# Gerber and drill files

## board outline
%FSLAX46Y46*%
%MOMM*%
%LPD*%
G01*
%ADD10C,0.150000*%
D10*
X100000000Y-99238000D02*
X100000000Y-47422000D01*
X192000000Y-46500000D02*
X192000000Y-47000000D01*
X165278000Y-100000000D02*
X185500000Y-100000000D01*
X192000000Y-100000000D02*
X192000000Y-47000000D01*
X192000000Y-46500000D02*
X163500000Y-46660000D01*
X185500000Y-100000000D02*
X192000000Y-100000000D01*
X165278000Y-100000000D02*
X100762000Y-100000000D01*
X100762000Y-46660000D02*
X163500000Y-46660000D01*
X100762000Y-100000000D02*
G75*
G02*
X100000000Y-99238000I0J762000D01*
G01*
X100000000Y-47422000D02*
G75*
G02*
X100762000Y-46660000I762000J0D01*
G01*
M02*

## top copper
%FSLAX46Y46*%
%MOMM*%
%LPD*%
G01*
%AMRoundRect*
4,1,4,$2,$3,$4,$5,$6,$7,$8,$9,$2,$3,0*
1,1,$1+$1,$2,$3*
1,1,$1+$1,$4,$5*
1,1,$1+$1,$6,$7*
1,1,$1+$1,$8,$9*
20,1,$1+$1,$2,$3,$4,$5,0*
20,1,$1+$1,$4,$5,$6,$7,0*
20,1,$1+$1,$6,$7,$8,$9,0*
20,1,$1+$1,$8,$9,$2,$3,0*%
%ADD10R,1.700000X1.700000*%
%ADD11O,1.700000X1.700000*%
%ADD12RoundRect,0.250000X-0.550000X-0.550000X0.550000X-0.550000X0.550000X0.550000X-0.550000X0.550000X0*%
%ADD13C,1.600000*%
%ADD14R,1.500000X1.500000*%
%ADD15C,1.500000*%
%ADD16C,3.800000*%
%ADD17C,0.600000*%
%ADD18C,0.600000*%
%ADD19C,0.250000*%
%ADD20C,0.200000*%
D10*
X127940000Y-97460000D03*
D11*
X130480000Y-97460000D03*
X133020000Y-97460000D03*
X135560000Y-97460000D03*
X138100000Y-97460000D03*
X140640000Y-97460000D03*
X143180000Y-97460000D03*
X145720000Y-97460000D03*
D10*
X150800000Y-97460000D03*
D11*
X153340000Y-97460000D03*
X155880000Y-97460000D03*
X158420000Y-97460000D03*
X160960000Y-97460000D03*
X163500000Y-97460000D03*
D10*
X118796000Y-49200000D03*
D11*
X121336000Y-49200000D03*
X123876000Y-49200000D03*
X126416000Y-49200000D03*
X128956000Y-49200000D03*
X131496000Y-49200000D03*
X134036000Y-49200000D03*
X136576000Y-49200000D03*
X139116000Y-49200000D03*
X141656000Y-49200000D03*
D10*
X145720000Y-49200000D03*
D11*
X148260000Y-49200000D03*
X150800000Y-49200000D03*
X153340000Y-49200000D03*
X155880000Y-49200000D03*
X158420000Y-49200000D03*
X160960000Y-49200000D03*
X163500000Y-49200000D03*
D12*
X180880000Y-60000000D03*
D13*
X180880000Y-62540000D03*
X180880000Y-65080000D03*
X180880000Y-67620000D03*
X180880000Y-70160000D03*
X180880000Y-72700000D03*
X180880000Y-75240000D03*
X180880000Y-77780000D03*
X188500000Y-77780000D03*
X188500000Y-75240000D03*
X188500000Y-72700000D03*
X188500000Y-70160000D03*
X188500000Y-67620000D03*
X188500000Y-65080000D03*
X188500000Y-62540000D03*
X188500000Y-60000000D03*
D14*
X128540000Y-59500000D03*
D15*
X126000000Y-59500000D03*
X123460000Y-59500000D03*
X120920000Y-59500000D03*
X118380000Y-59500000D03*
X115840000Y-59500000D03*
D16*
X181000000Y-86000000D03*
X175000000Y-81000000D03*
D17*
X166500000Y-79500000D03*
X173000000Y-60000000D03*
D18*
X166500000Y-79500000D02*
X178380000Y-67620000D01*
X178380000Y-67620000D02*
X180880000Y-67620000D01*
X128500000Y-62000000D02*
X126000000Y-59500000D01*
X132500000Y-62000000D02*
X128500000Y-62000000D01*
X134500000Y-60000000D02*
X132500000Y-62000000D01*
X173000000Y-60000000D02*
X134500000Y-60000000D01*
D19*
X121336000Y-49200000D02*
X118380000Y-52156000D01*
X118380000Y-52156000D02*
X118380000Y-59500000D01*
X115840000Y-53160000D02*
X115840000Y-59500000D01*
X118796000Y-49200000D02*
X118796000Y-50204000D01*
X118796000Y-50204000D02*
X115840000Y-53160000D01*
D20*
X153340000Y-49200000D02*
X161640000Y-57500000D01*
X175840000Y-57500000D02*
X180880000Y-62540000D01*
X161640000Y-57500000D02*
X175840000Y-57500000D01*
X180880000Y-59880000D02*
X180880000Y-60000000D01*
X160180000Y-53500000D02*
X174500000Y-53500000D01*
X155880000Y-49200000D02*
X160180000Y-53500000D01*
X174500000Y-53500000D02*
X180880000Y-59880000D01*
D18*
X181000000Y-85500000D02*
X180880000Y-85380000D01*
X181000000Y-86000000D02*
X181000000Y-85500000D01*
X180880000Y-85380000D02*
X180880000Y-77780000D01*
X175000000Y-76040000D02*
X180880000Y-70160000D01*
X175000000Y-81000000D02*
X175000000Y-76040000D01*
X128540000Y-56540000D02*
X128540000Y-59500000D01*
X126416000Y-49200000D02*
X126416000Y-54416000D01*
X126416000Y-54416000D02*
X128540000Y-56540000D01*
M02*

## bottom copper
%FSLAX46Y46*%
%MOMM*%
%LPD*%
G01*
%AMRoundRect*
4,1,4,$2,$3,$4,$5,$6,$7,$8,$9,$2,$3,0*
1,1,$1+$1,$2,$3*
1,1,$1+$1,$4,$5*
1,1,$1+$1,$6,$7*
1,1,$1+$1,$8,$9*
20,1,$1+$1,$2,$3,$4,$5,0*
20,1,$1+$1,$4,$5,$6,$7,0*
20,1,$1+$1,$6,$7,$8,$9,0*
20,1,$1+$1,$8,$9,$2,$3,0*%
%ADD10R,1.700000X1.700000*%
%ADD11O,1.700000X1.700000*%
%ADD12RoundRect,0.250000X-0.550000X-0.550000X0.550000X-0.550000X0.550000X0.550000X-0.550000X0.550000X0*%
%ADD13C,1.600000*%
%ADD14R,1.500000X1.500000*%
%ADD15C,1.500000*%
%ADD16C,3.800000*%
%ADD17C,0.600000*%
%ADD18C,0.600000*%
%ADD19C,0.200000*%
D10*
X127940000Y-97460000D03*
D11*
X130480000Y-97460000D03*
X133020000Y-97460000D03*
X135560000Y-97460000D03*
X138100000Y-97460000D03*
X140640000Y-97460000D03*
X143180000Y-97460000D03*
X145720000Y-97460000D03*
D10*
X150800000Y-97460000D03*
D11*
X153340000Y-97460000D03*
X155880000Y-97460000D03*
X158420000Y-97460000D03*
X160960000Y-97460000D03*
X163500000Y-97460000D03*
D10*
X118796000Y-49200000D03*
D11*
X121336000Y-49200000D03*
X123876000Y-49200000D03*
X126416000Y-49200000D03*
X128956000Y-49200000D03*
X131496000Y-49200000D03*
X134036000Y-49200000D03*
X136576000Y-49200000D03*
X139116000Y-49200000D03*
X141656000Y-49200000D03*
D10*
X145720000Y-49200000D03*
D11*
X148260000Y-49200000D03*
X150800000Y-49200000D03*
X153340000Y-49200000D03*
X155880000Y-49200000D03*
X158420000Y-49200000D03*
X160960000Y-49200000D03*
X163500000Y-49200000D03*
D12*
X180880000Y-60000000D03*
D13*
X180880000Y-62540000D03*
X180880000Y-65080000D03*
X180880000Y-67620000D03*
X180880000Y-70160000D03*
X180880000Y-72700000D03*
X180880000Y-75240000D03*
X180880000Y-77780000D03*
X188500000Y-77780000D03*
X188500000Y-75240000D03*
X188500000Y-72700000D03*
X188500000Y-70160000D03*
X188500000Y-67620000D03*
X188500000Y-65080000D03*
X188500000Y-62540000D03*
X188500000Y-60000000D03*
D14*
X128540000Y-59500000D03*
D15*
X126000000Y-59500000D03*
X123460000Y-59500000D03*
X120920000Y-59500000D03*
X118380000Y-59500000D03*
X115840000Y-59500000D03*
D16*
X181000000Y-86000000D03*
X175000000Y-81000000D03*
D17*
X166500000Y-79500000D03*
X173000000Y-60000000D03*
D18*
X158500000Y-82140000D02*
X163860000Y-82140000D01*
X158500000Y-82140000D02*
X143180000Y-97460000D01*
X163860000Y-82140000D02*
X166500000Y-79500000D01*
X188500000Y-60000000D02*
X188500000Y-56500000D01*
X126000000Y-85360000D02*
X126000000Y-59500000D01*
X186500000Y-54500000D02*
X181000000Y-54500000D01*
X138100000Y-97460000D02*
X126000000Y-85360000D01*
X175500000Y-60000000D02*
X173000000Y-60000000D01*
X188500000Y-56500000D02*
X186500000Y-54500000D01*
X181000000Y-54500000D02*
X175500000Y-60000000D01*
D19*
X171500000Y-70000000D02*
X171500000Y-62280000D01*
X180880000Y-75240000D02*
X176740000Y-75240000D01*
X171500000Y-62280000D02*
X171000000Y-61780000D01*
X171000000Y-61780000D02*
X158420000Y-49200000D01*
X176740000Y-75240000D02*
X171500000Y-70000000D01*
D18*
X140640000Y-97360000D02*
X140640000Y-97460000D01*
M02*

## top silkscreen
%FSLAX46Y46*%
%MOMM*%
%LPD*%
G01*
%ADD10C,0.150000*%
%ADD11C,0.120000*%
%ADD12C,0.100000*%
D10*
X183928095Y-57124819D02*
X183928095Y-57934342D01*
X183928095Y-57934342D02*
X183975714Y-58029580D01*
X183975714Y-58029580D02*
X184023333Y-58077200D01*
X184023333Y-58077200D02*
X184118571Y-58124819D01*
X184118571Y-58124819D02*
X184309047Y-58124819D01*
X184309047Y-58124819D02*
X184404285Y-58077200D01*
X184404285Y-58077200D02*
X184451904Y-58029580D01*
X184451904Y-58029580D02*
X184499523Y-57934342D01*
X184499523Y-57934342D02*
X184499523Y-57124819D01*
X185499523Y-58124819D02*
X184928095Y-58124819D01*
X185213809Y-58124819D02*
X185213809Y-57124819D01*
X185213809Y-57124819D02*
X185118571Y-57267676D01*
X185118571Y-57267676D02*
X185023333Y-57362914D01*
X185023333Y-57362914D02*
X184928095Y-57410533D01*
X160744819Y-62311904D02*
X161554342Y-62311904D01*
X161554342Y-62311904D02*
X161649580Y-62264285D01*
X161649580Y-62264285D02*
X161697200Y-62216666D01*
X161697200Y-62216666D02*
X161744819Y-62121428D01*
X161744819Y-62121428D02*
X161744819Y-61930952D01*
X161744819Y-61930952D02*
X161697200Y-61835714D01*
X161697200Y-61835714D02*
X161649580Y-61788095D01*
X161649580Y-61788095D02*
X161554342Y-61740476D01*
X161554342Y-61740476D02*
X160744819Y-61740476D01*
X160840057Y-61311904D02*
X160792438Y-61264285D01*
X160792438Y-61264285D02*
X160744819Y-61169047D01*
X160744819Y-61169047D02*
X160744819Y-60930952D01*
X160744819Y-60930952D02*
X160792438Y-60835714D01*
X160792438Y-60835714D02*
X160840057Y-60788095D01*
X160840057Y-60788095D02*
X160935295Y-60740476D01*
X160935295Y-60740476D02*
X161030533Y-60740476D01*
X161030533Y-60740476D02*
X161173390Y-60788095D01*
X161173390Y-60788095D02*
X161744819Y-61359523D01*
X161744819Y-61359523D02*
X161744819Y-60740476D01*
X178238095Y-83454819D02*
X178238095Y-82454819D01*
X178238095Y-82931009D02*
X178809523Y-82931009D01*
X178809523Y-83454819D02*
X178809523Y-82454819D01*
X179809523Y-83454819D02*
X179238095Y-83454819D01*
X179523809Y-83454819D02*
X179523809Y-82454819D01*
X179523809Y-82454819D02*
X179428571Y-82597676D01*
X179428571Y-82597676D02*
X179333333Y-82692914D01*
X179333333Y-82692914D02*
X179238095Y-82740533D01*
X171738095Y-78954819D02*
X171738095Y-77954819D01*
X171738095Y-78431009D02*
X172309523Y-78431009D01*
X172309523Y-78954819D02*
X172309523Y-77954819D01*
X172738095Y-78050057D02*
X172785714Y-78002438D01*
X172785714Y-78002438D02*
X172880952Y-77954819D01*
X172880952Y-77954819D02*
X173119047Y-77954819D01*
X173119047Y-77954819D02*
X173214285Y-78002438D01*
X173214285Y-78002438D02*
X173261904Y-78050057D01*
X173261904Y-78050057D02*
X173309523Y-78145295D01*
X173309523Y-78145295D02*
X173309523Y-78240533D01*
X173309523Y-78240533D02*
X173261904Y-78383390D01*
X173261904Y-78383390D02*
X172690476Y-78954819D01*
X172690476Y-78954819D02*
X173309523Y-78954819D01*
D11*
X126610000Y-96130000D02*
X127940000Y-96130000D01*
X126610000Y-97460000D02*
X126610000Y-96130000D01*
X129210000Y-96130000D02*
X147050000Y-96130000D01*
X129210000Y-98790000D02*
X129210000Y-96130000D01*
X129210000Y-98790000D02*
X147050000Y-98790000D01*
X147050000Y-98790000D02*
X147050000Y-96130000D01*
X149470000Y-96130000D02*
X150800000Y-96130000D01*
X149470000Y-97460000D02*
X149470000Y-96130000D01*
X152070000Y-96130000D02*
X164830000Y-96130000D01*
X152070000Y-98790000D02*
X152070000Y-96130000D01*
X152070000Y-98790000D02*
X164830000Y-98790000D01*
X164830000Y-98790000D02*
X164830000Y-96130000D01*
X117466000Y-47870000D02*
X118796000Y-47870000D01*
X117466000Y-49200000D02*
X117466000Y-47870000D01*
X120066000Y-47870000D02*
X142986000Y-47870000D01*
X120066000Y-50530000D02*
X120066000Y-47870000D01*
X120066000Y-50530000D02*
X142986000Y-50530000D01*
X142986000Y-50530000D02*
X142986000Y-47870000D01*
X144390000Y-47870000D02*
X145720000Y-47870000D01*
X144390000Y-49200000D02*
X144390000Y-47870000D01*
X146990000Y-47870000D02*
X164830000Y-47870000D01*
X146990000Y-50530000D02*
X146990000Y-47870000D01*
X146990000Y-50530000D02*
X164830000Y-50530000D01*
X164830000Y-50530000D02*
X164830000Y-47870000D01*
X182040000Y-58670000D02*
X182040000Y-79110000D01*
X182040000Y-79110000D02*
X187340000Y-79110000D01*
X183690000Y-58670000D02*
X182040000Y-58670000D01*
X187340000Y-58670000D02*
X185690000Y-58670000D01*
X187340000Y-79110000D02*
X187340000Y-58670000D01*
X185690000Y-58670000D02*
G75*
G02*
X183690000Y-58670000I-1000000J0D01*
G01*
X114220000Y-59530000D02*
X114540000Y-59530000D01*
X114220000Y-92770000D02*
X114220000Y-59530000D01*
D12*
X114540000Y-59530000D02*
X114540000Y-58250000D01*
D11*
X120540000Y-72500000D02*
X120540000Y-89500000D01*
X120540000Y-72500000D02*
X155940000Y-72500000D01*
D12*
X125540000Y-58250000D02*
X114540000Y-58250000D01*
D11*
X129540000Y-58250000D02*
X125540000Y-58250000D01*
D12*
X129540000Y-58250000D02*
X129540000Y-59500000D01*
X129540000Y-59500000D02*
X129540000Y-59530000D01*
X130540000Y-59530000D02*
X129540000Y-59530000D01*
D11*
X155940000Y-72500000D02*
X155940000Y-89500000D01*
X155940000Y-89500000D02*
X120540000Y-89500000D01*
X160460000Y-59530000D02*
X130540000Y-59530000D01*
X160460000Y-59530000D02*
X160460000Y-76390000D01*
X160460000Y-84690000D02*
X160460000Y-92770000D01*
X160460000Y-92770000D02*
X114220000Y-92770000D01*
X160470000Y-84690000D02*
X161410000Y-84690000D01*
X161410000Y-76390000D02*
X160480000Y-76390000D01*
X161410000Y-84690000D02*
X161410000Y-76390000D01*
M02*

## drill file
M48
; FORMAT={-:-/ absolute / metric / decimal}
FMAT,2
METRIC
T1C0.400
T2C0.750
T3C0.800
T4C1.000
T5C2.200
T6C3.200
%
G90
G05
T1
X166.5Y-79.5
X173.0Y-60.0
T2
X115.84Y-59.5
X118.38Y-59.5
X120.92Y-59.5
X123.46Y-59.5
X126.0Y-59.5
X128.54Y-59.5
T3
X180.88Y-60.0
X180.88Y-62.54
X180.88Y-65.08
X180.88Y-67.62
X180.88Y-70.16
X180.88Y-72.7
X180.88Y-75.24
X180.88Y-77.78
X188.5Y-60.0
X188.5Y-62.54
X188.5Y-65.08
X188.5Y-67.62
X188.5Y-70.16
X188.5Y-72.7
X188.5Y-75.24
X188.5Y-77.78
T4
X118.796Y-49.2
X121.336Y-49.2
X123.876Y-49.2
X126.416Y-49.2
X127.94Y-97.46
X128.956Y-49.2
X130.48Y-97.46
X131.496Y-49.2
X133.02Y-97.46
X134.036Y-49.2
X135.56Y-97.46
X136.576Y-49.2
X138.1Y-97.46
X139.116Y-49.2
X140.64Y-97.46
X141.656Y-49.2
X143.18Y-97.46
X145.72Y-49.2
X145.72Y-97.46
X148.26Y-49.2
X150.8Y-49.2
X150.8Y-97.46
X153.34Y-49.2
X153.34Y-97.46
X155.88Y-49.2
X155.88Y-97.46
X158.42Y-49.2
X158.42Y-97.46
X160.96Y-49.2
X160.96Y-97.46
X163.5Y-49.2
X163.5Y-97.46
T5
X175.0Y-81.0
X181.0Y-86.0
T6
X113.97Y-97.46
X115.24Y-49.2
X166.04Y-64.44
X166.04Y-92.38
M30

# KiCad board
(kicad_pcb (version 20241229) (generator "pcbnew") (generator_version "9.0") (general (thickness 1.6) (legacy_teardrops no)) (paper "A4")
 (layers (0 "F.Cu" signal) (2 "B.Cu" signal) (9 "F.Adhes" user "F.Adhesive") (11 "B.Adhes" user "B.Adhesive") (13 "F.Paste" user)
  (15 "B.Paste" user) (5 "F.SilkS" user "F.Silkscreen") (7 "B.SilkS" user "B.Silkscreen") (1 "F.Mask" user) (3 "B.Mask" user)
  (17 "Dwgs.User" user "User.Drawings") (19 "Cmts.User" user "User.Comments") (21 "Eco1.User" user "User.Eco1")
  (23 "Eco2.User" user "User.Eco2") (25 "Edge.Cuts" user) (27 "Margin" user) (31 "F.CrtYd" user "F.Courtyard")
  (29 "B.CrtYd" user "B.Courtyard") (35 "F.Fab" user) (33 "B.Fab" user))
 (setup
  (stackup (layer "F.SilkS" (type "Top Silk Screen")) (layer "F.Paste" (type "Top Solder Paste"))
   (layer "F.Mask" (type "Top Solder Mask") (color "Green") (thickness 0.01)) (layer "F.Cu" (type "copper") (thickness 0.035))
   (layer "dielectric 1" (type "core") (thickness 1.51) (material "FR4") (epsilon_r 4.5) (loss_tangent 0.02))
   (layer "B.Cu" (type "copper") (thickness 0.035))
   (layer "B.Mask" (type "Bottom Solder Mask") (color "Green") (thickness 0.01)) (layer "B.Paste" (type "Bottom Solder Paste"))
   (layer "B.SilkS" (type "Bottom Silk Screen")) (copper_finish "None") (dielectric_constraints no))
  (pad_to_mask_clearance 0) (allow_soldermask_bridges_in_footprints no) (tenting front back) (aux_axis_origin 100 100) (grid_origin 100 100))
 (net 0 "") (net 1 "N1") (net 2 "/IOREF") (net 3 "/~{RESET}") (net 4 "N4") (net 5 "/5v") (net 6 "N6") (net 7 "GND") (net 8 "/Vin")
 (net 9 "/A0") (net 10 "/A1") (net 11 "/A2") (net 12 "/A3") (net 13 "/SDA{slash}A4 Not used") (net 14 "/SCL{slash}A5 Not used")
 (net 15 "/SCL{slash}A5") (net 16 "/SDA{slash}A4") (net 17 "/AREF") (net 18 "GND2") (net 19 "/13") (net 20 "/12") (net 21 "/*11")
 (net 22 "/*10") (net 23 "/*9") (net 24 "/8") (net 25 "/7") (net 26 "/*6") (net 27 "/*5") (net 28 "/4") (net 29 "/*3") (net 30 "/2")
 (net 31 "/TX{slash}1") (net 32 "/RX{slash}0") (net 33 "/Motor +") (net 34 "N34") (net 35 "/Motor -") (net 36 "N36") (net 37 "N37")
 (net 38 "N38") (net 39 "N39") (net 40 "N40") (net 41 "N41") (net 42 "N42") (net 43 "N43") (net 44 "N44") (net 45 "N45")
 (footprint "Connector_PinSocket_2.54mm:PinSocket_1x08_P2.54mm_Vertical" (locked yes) (layer "F.Cu") (at 127.94 97.46 90)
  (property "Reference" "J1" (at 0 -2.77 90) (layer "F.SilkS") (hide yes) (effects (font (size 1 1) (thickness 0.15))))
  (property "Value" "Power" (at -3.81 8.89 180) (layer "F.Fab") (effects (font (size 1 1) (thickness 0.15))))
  (fp_line (start 1.33 -1.33) (end 1.33 0) (stroke (width 0.12) (type solid)) (layer "F.SilkS"))
  (fp_line (start 0 -1.33) (end 1.33 -1.33) (stroke (width 0.12) (type solid)) (layer "F.SilkS"))
  (fp_line (start 1.33 1.27) (end 1.33 19.11) (stroke (width 0.12) (type solid)) (layer "F.SilkS"))
  (fp_line (start -1.33 1.27) (end 1.33 1.27) (stroke (width 0.12) (type solid)) (layer "F.SilkS"))
  (fp_line (start -1.33 1.27) (end -1.33 19.11) (stroke (width 0.12) (type solid)) (layer "F.SilkS"))
  (fp_line (start -1.33 19.11) (end 1.33 19.11) (stroke (width 0.12) (type solid)) (layer "F.SilkS"))
  (pad "1" thru_hole rect (at 0 0 90) (size 1.7 1.7) (drill 1) (layers "*.Cu" "*.Mask") (remove_unused_layers no) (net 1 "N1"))
  (pad "2" thru_hole oval (at 0 2.54 90) (size 1.7 1.7) (drill 1) (layers "*.Cu" "*.Mask") (remove_unused_layers no) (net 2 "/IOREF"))
  (pad "3" thru_hole oval (at 0 5.08 90) (size 1.7 1.7) (drill 1) (layers "*.Cu" "*.Mask") (remove_unused_layers no) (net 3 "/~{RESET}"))
  (pad "4" thru_hole oval (at 0 7.62 90) (size 1.7 1.7) (drill 1) (layers "*.Cu" "*.Mask") (remove_unused_layers no) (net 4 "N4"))
  (pad "5" thru_hole oval (at 0 10.16 90) (size 1.7 1.7) (drill 1) (layers "*.Cu" "*.Mask") (remove_unused_layers no) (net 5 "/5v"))
  (pad "6" thru_hole oval (at 0 12.7 90) (size 1.7 1.7) (drill 1) (layers "*.Cu" "*.Mask") (remove_unused_layers no) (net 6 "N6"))
  (pad "7" thru_hole oval (at 0 15.24 90) (size 1.7 1.7) (drill 1) (layers "*.Cu" "*.Mask") (remove_unused_layers no) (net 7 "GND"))
  (pad "8" thru_hole oval (at 0 17.78 90) (size 1.7 1.7) (drill 1) (layers "*.Cu" "*.Mask") (remove_unused_layers no) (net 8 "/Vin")))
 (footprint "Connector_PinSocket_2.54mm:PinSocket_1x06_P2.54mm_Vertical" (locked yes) (layer "F.Cu") (at 150.8 97.46 90)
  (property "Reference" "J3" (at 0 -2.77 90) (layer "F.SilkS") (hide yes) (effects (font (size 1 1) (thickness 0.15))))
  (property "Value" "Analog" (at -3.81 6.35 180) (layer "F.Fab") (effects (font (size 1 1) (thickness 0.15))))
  (fp_line (start 1.33 -1.33) (end 1.33 0) (stroke (width 0.12) (type solid)) (layer "F.SilkS"))
  (fp_line (start 0 -1.33) (end 1.33 -1.33) (stroke (width 0.12) (type solid)) (layer "F.SilkS"))
  (fp_line (start 1.33 1.27) (end 1.33 14.03) (stroke (width 0.12) (type solid)) (layer "F.SilkS"))
  (fp_line (start -1.33 1.27) (end 1.33 1.27) (stroke (width 0.12) (type solid)) (layer "F.SilkS"))
  (fp_line (start -1.33 1.27) (end -1.33 14.03) (stroke (width 0.12) (type solid)) (layer "F.SilkS"))
  (fp_line (start -1.33 14.03) (end 1.33 14.03) (stroke (width 0.12) (type solid)) (layer "F.SilkS"))
  (pad "1" thru_hole rect (at 0 0 90) (size 1.7 1.7) (drill 1) (layers "*.Cu" "*.Mask") (remove_unused_layers no) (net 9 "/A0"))
  (pad "2" thru_hole oval (at 0 2.54 90) (size 1.7 1.7) (drill 1) (layers "*.Cu" "*.Mask") (remove_unused_layers no) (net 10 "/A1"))
  (pad "3" thru_hole oval (at 0 5.08 90) (size 1.7 1.7) (drill 1) (layers "*.Cu" "*.Mask") (remove_unused_layers no) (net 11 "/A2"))
  (pad "4" thru_hole oval (at 0 7.62 90) (size 1.7 1.7) (drill 1) (layers "*.Cu" "*.Mask") (remove_unused_layers no) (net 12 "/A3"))
  (pad "5" thru_hole oval (at 0 10.16 90) (size 1.7 1.7) (drill 1) (layers "*.Cu" "*.Mask") (remove_unused_layers no)
   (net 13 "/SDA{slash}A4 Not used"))
  (pad "6" thru_hole oval (at 0 12.7 90) (size 1.7 1.7) (drill 1) (layers "*.Cu" "*.Mask") (remove_unused_layers no)
   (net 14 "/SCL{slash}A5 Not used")))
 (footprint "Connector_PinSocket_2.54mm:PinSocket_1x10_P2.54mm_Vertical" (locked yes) (layer "F.Cu") (at 118.796 49.2 90)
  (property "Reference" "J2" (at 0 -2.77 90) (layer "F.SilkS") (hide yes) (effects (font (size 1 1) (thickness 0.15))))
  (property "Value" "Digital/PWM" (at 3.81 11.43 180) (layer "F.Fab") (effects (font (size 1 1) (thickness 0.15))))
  (fp_line (start 1.33 -1.33) (end 1.33 0) (stroke (width 0.12) (type solid)) (layer "F.SilkS"))
  (fp_line (start 0 -1.33) (end 1.33 -1.33) (stroke (width 0.12) (type solid)) (layer "F.SilkS"))
  (fp_line (start 1.33 1.27) (end 1.33 24.19) (stroke (width 0.12) (type solid)) (layer "F.SilkS"))
  (fp_line (start -1.33 1.27) (end 1.33 1.27) (stroke (width 0.12) (type solid)) (layer "F.SilkS"))
  (fp_line (start -1.33 1.27) (end -1.33 24.19) (stroke (width 0.12) (type solid)) (layer "F.SilkS"))
  (fp_line (start -1.33 24.19) (end 1.33 24.19) (stroke (width 0.12) (type solid)) (layer "F.SilkS"))
  (pad "1" thru_hole rect (at 0 0 90) (size 1.7 1.7) (drill 1) (layers "*.Cu" "*.Mask") (remove_unused_layers no) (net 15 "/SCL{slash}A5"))
  (pad "2" thru_hole oval (at 0 2.54 90) (size 1.7 1.7) (drill 1) (layers "*.Cu" "*.Mask") (remove_unused_layers no)
   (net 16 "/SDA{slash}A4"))
  (pad "3" thru_hole oval (at 0 5.08 90) (size 1.7 1.7) (drill 1) (layers "*.Cu" "*.Mask") (remove_unused_layers no) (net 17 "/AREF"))
  (pad "4" thru_hole oval (at 0 7.62 90) (size 1.7 1.7) (drill 1) (layers "*.Cu" "*.Mask") (remove_unused_layers no) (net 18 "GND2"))
  (pad "5" thru_hole oval (at 0 10.16 90) (size 1.7 1.7) (drill 1) (layers "*.Cu" "*.Mask") (remove_unused_layers no) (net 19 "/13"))
  (pad "6" thru_hole oval (at 0 12.7 90) (size 1.7 1.7) (drill 1) (layers "*.Cu" "*.Mask") (remove_unused_layers no) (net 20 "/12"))
  (pad "7" thru_hole oval (at 0 15.24 90) (size 1.7 1.7) (drill 1) (layers "*.Cu" "*.Mask") (remove_unused_layers no) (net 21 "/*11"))
  (pad "8" thru_hole oval (at 0 17.78 90) (size 1.7 1.7) (drill 1) (layers "*.Cu" "*.Mask") (remove_unused_layers no) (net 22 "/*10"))
  (pad "9" thru_hole oval (at 0 20.32 90) (size 1.7 1.7) (drill 1) (layers "*.Cu" "*.Mask") (remove_unused_layers no) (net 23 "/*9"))
  (pad "10" thru_hole oval (at 0 22.86 90) (size 1.7 1.7) (drill 1) (layers "*.Cu" "*.Mask") (remove_unused_layers no) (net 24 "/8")))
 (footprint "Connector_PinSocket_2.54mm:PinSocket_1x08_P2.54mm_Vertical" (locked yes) (layer "F.Cu") (at 145.72 49.2 90)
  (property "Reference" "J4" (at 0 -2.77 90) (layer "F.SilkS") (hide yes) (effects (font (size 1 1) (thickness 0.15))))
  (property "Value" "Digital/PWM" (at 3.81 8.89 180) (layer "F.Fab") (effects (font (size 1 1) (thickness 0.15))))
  (fp_line (start 1.33 -1.33) (end 1.33 0) (stroke (width 0.12) (type solid)) (layer "F.SilkS"))
  (fp_line (start 0 -1.33) (end 1.33 -1.33) (stroke (width 0.12) (type solid)) (layer "F.SilkS"))
  (fp_line (start 1.33 1.27) (end 1.33 19.11) (stroke (width 0.12) (type solid)) (layer "F.SilkS"))
  (fp_line (start -1.33 1.27) (end 1.33 1.27) (stroke (width 0.12) (type solid)) (layer "F.SilkS"))
  (fp_line (start -1.33 1.27) (end -1.33 19.11) (stroke (width 0.12) (type solid)) (layer "F.SilkS"))
  (fp_line (start -1.33 19.11) (end 1.33 19.11) (stroke (width 0.12) (type solid)) (layer "F.SilkS"))
  (pad "1" thru_hole rect (at 0 0 90) (size 1.7 1.7) (drill 1) (layers "*.Cu" "*.Mask") (remove_unused_layers no) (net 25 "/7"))
  (pad "2" thru_hole oval (at 0 2.54 90) (size 1.7 1.7) (drill 1) (layers "*.Cu" "*.Mask") (remove_unused_layers no) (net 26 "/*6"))
  (pad "3" thru_hole oval (at 0 5.08 90) (size 1.7 1.7) (drill 1) (layers "*.Cu" "*.Mask") (remove_unused_layers no) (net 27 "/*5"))
  (pad "4" thru_hole oval (at 0 7.62 90) (size 1.7 1.7) (drill 1) (layers "*.Cu" "*.Mask") (remove_unused_layers no) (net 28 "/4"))
  (pad "5" thru_hole oval (at 0 10.16 90) (size 1.7 1.7) (drill 1) (layers "*.Cu" "*.Mask") (remove_unused_layers no) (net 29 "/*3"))
  (pad "6" thru_hole oval (at 0 12.7 90) (size 1.7 1.7) (drill 1) (layers "*.Cu" "*.Mask") (remove_unused_layers no) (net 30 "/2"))
  (pad "7" thru_hole oval (at 0 15.24 90) (size 1.7 1.7) (drill 1) (layers "*.Cu" "*.Mask") (remove_unused_layers no) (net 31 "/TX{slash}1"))
  (pad "8" thru_hole oval (at 0 17.78 90) (size 1.7 1.7) (drill 1) (layers "*.Cu" "*.Mask") (remove_unused_layers no) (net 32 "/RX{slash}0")))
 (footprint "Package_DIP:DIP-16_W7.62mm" (layer "F.Cu") (at 180.88 60)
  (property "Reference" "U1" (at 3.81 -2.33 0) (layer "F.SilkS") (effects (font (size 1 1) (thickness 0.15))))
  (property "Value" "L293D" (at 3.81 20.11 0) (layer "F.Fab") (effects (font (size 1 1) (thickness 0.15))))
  (fp_line (start 1.16 -1.33) (end 1.16 19.11) (stroke (width 0.12) (type solid)) (layer "F.SilkS"))
  (fp_line (start 1.16 19.11) (end 6.46 19.11) (stroke (width 0.12) (type solid)) (layer "F.SilkS"))
  (fp_line (start 2.81 -1.33) (end 1.16 -1.33) (stroke (width 0.12) (type solid)) (layer "F.SilkS"))
  (fp_line (start 6.46 -1.33) (end 4.81 -1.33) (stroke (width 0.12) (type solid)) (layer "F.SilkS"))
  (fp_line (start 6.46 19.11) (end 6.46 -1.33) (stroke (width 0.12) (type solid)) (layer "F.SilkS"))
  (fp_arc (start 4.81 -1.33) (mid 3.81 -0.33) (end 2.81 -1.33) (stroke (width 0.12) (type solid)) (layer "F.SilkS"))
  (pad "1" thru_hole roundrect (at 0 0) (size 1.6 1.6) (drill 0.8) (layers "*.Cu" "*.Mask") (remove_unused_layers no)
   (roundrect_rratio 0.15625) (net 29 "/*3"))
  (pad "2" thru_hole circle (at 0 2.54) (size 1.6 1.6) (drill 0.8) (layers "*.Cu" "*.Mask") (remove_unused_layers no) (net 28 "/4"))
  (pad "3" thru_hole circle (at 0 5.08) (size 1.6 1.6) (drill 0.8) (layers "*.Cu" "*.Mask") (remove_unused_layers no) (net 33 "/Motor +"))
  (pad "4" thru_hole circle (at 0 7.62) (size 1.6 1.6) (drill 0.8) (layers "*.Cu" "*.Mask") (remove_unused_layers no) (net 7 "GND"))
  (pad "5" thru_hole circle (at 0 10.16) (size 1.6 1.6) (drill 0.8) (layers "*.Cu" "*.Mask") (remove_unused_layers no) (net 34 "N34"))
  (pad "6" thru_hole circle (at 0 12.7) (size 1.6 1.6) (drill 0.8) (layers "*.Cu" "*.Mask") (remove_unused_layers no) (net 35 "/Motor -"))
  (pad "7" thru_hole circle (at 0 15.24) (size 1.6 1.6) (drill 0.8) (layers "*.Cu" "*.Mask") (remove_unused_layers no) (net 30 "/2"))
  (pad "8" thru_hole circle (at 0 17.78) (size 1.6 1.6) (drill 0.8) (layers "*.Cu" "*.Mask") (remove_unused_layers no) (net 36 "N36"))
  (pad "9" thru_hole circle (at 7.62 17.78) (size 1.6 1.6) (drill 0.8) (layers "*.Cu" "*.Mask") (remove_unused_layers no) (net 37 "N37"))
  (pad "10" thru_hole circle (at 7.62 15.24) (size 1.6 1.6) (drill 0.8) (layers "*.Cu" "*.Mask") (remove_unused_layers no) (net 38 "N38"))
  (pad "11" thru_hole circle (at 7.62 12.7) (size 1.6 1.6) (drill 0.8) (layers "*.Cu" "*.Mask") (remove_unused_layers no) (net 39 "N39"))
  (pad "12" thru_hole circle (at 7.62 10.16) (size 1.6 1.6) (drill 0.8) (layers "*.Cu" "*.Mask") (remove_unused_layers no) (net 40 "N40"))
  (pad "13" thru_hole circle (at 7.62 7.62) (size 1.6 1.6) (drill 0.8) (layers "*.Cu" "*.Mask") (remove_unused_layers no) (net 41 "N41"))
  (pad "14" thru_hole circle (at 7.62 5.08) (size 1.6 1.6) (drill 0.8) (layers "*.Cu" "*.Mask") (remove_unused_layers no) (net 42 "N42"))
  (pad "15" thru_hole circle (at 7.62 2.54) (size 1.6 1.6) (drill 0.8) (layers "*.Cu" "*.Mask") (remove_unused_layers no) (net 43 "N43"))
  (pad "16" thru_hole circle (at 7.62 0) (size 1.6 1.6) (drill 0.8) (layers "*.Cu" "*.Mask") (remove_unused_layers no) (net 5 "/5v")))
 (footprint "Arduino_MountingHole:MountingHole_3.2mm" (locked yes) (layer "F.Cu") (at 115.24 49.2)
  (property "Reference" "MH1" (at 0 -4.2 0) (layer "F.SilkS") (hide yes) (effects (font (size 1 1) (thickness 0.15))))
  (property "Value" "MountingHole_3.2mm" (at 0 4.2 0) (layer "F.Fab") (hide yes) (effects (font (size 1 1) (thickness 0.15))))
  (pad "" np_thru_hole circle (at 0 0) (size 3.2 3.2) (drill 3.2) (layers "*.Cu" "*.Mask")))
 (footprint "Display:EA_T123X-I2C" (layer "F.Cu") (at 128.54 59.5 -90)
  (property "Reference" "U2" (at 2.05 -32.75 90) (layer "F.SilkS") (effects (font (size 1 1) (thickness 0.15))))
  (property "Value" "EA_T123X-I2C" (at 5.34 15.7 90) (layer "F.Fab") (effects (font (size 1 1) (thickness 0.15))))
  (fp_line (start 0.03 14.32) (end 0.03 14) (stroke (width 0.12) (type solid)) (layer "F.SilkS"))
  (fp_line (start 33.27 14.32) (end 0.03 14.32) (stroke (width 0.12) (type solid)) (layer "F.SilkS"))
  (fp_line (start 0.03 14) (end -1.25 14) (stroke (width 0.1) (type default)) (layer "F.SilkS"))
  (fp_line (start 13 8) (end 30 8) (stroke (width 0.12) (type solid)) (layer "F.SilkS"))
  (fp_line (start 13 8) (end 13 -27.4) (stroke (width 0.12) (type solid)) (layer "F.SilkS"))
  (fp_line (start -1.25 3) (end -1.25 14) (stroke (width 0.1) (type default)) (layer "F.SilkS"))
  (fp_line (start -1.25 -1) (end -1.25 3) (stroke (width 0.12) (type solid)) (layer "F.SilkS"))
  (fp_line (start -1.25 -1) (end 0 -1) (stroke (width 0.1) (type default)) (layer "F.SilkS"))
  (fp_line (start 0 -1) (end 0.03 -1) (stroke (width 0.1) (type default)) (layer "F.SilkS"))
  (fp_line (start 0.03 -2) (end 0.03 -1) (stroke (width 0.1) (type default)) (layer "F.SilkS"))
  (fp_line (start 13 -27.4) (end 30 -27.4) (stroke (width 0.12) (type solid)) (layer "F.SilkS"))
  (fp_line (start 30 -27.4) (end 30 8) (stroke (width 0.12) (type solid)) (layer "F.SilkS"))
  (fp_line (start 0.03 -31.92) (end 0.03 -2) (stroke (width 0.12) (type solid)) (layer "F.SilkS"))
  (fp_line (start 0.03 -31.92) (end 16.89 -31.92) (stroke (width 0.12) (type solid)) (layer "F.SilkS"))
  (fp_line (start 25.19 -31.92) (end 33.27 -31.92) (stroke (width 0.12) (type solid)) (layer "F.SilkS"))
  (fp_line (start 33.27 -31.92) (end 33.27 14.32) (stroke (width 0.12) (type solid)) (layer "F.SilkS"))
  (fp_line (start 25.19 -31.93) (end 25.19 -32.87) (stroke (width 0.12) (type solid)) (layer "F.SilkS"))
  (fp_line (start 16.89 -32.87) (end 16.89 -31.94) (stroke (width 0.12) (type solid)) (layer "F.SilkS"))
  (fp_line (start 25.19 -32.87) (end 16.89 -32.87) (stroke (width 0.12) (type solid)) (layer "F.SilkS"))
  (pad "1" thru_hole rect (at 0 0 270) (size 1.5 1.5) (drill 0.75) (layers "*.Cu" "*.Mask") (remove_unused_layers no) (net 18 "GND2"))
  (pad "2" thru_hole circle (at 0 2.54 270) (size 1.5 1.5) (drill 0.75) (layers "*.Cu" "*.Mask") (remove_unused_layers no) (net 5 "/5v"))
  (pad "3" thru_hole circle (at 0 5.08 270) (size 1.5 1.5) (drill 0.75) (layers "*.Cu" "*.Mask") (remove_unused_layers no) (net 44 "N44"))
  (pad "4" thru_hole circle (at 0 7.62 270) (size 1.5 1.5) (drill 0.75) (layers "*.Cu" "*.Mask") (remove_unused_layers no) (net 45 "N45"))
  (pad "5" thru_hole circle (at 0 10.16 270) (size 1.5 1.5) (drill 0.75) (layers "*.Cu" "*.Mask") (remove_unused_layers no)
   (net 16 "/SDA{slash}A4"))
  (pad "6" thru_hole circle (at 0 12.7 270) (size 1.5 1.5) (drill 0.75) (layers "*.Cu" "*.Mask") (remove_unused_layers no)
   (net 15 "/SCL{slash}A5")))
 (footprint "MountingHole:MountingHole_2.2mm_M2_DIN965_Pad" (layer "F.Cu") (at 181 86)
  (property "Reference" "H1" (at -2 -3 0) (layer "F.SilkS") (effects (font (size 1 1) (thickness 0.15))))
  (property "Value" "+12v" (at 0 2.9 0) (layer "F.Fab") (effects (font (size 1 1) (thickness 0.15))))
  (pad "1" thru_hole circle (at 0 0) (size 3.8 3.8) (drill 2.2) (layers "*.Cu" "*.Mask") (remove_unused_layers no) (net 36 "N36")))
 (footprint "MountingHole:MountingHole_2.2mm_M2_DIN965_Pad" (layer "F.Cu") (at 175 81)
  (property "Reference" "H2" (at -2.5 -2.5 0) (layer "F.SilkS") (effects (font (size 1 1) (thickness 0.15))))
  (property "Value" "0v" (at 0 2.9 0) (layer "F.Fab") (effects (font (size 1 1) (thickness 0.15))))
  (pad "1" thru_hole circle (at 0 0) (size 3.8 3.8) (drill 2.2) (layers "*.Cu" "*.Mask") (remove_unused_layers no) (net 34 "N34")))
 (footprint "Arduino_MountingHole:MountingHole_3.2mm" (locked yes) (layer "F.Cu") (at 113.97 97.46)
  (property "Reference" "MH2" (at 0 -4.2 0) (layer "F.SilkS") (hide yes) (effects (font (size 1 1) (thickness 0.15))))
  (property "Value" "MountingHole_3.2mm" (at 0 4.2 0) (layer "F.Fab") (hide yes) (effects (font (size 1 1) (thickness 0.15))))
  (pad "" np_thru_hole circle (at 0 0) (size 3.2 3.2) (drill 3.2) (layers "*.Cu" "*.Mask")))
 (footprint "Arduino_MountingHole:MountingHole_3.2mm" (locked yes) (layer "F.Cu") (at 166.04 64.44)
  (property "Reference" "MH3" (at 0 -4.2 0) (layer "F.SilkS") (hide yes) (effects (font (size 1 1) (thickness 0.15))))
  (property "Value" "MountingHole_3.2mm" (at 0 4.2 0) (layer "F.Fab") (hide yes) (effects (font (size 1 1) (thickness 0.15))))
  (pad "" np_thru_hole circle (at 0 0) (size 3.2 3.2) (drill 3.2) (layers "*.Cu" "*.Mask")))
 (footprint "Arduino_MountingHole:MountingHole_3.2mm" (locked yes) (layer "F.Cu") (at 166.04 92.38)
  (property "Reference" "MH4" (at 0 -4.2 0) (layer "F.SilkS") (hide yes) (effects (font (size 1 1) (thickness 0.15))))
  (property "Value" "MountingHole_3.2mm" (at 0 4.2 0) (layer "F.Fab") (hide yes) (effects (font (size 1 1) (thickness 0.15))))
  (pad "" np_thru_hole circle (at 0 0) (size 3.2 3.2) (drill 3.2) (layers "*.Cu" "*.Mask")))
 (gr_line (start 100 99.238) (end 100 47.422) (stroke (width 0.15) (type solid)) (layer "Edge.Cuts"))
 (gr_line (start 192 46.5) (end 192 47) (stroke (width 0.15) (type default)) (layer "Edge.Cuts"))
 (gr_line (start 165.278 100) (end 185.5 100) (stroke (width 0.15) (type default)) (layer "Edge.Cuts"))
 (gr_line (start 192 100) (end 192 47) (stroke (width 0.15) (type default)) (layer "Edge.Cuts"))
 (gr_line (start 192 46.5) (end 163.5 46.66) (stroke (width 0.15) (type default)) (layer "Edge.Cuts"))
 (gr_line (start 185.5 100) (end 192 100) (stroke (width 0.15) (type default)) (layer "Edge.Cuts"))
 (gr_line (start 165.278 100) (end 100.762 100) (stroke (width 0.15) (type solid)) (layer "Edge.Cuts"))
 (gr_line (start 100.762 46.66) (end 163.5 46.66) (stroke (width 0.15) (type solid)) (layer "Edge.Cuts"))
 (gr_arc (start 100.762 100) (mid 100.223185 99.776815) (end 100 99.238) (stroke (width 0.15) (type solid)) (layer "Edge.Cuts"))
 (gr_arc (start 100 47.422) (mid 100.223185 46.883185) (end 100.762 46.66) (stroke (width 0.15) (type solid)) (layer "Edge.Cuts"))
 (segment (start 166.5 79.5) (end 178.38 67.62) (width 0.6) (layer "F.Cu") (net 7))
 (segment (start 178.38 67.62) (end 180.88 67.62) (width 0.6) (layer "F.Cu") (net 7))
 (via (at 166.5 79.5) (size 0.6) (drill 0.4) (layers "F.Cu" "B.Cu") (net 7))
 (segment (start 158.5 82.14) (end 163.86 82.14) (width 0.6) (layer "B.Cu") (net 7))
 (segment (start 158.5 82.14) (end 143.18 97.46) (width 0.6) (layer "B.Cu") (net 7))
 (segment (start 163.86 82.14) (end 166.5 79.5) (width 0.6) (layer "B.Cu") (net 7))
 (segment (start 128.5 62) (end 126 59.5) (width 0.6) (layer "F.Cu") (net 5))
 (segment (start 132.5 62) (end 128.5 62) (width 0.6) (layer "F.Cu") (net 5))
 (segment (start 134.5 60) (end 132.5 62) (width 0.6) (layer "F.Cu") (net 5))
 (segment (start 173 60) (end 134.5 60) (width 0.6) (layer "F.Cu") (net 5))
 (via (at 173 60) (size 0.6) (drill 0.4) (layers "F.Cu" "B.Cu") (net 5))
 (segment (start 188.5 60) (end 188.5 56.5) (width 0.6) (layer "B.Cu") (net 5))
 (segment (start 126 85.36) (end 126 59.5) (width 0.6) (layer "B.Cu") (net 5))
 (segment (start 186.5 54.5) (end 181 54.5) (width 0.6) (layer "B.Cu") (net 5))
 (segment (start 138.1 97.46) (end 126 85.36) (width 0.6) (layer "B.Cu") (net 5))
 (segment (start 175.5 60) (end 173 60) (width 0.6) (layer "B.Cu") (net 5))
 (segment (start 188.5 56.5) (end 186.5 54.5) (width 0.6) (layer "B.Cu") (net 5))
 (segment (start 181 54.5) (end 175.5 60) (width 0.6) (layer "B.Cu") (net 5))
 (segment (start 121.336 49.2) (end 118.38 52.156) (width 0.25) (layer "F.Cu") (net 16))
 (segment (start 118.38 52.156) (end 118.38 59.5) (width 0.25) (layer "F.Cu") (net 16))
 (segment (start 115.84 53.16) (end 115.84 59.5) (width 0.25) (layer "F.Cu") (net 15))
 (segment (start 118.796 49.2) (end 118.796 50.204) (width 0.25) (layer "F.Cu") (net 15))
 (segment (start 118.796 50.204) (end 115.84 53.16) (width 0.25) (layer "F.Cu") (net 15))
 (segment (start 153.34 49.2) (end 161.64 57.5) (width 0.2) (layer "F.Cu") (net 28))
 (segment (start 175.84 57.5) (end 180.88 62.54) (width 0.2) (layer "F.Cu") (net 28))
 (segment (start 161.64 57.5) (end 175.84 57.5) (width 0.2) (layer "F.Cu") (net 28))
 (segment (start 171.5 70) (end 171.5 62.28) (width 0.2) (layer "B.Cu") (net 30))
 (segment (start 180.88 75.24) (end 176.74 75.24) (width 0.2) (layer "B.Cu") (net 30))
 (segment (start 171.5 62.28) (end 171 61.78) (width 0.2) (layer "B.Cu") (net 30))
 (segment (start 171 61.78) (end 158.42 49.2) (width 0.2) (layer "B.Cu") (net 30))
 (segment (start 176.74 75.24) (end 171.5 70) (width 0.2) (layer "B.Cu") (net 30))
 (segment (start 180.88 59.88) (end 180.88 60) (width 0.2) (layer "F.Cu") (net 29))
 (segment (start 160.18 53.5) (end 174.5 53.5) (width 0.2) (layer "F.Cu") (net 29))
 (segment (start 155.88 49.2) (end 160.18 53.5) (width 0.2) (layer "F.Cu") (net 29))
 (segment (start 174.5 53.5) (end 180.88 59.88) (width 0.2) (layer "F.Cu") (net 29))
 (segment (start 181 85.5) (end 180.88 85.38) (width 0.6) (layer "F.Cu") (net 36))
 (segment (start 181 86) (end 181 85.5) (width 0.6) (layer "F.Cu") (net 36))
 (segment (start 180.88 85.38) (end 180.88 77.78) (width 0.6) (layer "F.Cu") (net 36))
 (segment (start 175 76.04) (end 180.88 70.16) (width 0.6) (layer "F.Cu") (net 34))
 (segment (start 175 81) (end 175 76.04) (width 0.6) (layer "F.Cu") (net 34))
 (segment (start 128.54 56.54) (end 128.54 59.5) (width 0.6) (layer "F.Cu") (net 18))
 (segment (start 126.416 49.2) (end 126.416 54.416) (width 0.6) (layer "F.Cu") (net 18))
 (segment (start 126.416 54.416) (end 128.54 56.54) (width 0.6) (layer "F.Cu") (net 18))
 (segment (start 140.64 97.36) (end 140.64 97.46) (width 0.6) (layer "B.Cu") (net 6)))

